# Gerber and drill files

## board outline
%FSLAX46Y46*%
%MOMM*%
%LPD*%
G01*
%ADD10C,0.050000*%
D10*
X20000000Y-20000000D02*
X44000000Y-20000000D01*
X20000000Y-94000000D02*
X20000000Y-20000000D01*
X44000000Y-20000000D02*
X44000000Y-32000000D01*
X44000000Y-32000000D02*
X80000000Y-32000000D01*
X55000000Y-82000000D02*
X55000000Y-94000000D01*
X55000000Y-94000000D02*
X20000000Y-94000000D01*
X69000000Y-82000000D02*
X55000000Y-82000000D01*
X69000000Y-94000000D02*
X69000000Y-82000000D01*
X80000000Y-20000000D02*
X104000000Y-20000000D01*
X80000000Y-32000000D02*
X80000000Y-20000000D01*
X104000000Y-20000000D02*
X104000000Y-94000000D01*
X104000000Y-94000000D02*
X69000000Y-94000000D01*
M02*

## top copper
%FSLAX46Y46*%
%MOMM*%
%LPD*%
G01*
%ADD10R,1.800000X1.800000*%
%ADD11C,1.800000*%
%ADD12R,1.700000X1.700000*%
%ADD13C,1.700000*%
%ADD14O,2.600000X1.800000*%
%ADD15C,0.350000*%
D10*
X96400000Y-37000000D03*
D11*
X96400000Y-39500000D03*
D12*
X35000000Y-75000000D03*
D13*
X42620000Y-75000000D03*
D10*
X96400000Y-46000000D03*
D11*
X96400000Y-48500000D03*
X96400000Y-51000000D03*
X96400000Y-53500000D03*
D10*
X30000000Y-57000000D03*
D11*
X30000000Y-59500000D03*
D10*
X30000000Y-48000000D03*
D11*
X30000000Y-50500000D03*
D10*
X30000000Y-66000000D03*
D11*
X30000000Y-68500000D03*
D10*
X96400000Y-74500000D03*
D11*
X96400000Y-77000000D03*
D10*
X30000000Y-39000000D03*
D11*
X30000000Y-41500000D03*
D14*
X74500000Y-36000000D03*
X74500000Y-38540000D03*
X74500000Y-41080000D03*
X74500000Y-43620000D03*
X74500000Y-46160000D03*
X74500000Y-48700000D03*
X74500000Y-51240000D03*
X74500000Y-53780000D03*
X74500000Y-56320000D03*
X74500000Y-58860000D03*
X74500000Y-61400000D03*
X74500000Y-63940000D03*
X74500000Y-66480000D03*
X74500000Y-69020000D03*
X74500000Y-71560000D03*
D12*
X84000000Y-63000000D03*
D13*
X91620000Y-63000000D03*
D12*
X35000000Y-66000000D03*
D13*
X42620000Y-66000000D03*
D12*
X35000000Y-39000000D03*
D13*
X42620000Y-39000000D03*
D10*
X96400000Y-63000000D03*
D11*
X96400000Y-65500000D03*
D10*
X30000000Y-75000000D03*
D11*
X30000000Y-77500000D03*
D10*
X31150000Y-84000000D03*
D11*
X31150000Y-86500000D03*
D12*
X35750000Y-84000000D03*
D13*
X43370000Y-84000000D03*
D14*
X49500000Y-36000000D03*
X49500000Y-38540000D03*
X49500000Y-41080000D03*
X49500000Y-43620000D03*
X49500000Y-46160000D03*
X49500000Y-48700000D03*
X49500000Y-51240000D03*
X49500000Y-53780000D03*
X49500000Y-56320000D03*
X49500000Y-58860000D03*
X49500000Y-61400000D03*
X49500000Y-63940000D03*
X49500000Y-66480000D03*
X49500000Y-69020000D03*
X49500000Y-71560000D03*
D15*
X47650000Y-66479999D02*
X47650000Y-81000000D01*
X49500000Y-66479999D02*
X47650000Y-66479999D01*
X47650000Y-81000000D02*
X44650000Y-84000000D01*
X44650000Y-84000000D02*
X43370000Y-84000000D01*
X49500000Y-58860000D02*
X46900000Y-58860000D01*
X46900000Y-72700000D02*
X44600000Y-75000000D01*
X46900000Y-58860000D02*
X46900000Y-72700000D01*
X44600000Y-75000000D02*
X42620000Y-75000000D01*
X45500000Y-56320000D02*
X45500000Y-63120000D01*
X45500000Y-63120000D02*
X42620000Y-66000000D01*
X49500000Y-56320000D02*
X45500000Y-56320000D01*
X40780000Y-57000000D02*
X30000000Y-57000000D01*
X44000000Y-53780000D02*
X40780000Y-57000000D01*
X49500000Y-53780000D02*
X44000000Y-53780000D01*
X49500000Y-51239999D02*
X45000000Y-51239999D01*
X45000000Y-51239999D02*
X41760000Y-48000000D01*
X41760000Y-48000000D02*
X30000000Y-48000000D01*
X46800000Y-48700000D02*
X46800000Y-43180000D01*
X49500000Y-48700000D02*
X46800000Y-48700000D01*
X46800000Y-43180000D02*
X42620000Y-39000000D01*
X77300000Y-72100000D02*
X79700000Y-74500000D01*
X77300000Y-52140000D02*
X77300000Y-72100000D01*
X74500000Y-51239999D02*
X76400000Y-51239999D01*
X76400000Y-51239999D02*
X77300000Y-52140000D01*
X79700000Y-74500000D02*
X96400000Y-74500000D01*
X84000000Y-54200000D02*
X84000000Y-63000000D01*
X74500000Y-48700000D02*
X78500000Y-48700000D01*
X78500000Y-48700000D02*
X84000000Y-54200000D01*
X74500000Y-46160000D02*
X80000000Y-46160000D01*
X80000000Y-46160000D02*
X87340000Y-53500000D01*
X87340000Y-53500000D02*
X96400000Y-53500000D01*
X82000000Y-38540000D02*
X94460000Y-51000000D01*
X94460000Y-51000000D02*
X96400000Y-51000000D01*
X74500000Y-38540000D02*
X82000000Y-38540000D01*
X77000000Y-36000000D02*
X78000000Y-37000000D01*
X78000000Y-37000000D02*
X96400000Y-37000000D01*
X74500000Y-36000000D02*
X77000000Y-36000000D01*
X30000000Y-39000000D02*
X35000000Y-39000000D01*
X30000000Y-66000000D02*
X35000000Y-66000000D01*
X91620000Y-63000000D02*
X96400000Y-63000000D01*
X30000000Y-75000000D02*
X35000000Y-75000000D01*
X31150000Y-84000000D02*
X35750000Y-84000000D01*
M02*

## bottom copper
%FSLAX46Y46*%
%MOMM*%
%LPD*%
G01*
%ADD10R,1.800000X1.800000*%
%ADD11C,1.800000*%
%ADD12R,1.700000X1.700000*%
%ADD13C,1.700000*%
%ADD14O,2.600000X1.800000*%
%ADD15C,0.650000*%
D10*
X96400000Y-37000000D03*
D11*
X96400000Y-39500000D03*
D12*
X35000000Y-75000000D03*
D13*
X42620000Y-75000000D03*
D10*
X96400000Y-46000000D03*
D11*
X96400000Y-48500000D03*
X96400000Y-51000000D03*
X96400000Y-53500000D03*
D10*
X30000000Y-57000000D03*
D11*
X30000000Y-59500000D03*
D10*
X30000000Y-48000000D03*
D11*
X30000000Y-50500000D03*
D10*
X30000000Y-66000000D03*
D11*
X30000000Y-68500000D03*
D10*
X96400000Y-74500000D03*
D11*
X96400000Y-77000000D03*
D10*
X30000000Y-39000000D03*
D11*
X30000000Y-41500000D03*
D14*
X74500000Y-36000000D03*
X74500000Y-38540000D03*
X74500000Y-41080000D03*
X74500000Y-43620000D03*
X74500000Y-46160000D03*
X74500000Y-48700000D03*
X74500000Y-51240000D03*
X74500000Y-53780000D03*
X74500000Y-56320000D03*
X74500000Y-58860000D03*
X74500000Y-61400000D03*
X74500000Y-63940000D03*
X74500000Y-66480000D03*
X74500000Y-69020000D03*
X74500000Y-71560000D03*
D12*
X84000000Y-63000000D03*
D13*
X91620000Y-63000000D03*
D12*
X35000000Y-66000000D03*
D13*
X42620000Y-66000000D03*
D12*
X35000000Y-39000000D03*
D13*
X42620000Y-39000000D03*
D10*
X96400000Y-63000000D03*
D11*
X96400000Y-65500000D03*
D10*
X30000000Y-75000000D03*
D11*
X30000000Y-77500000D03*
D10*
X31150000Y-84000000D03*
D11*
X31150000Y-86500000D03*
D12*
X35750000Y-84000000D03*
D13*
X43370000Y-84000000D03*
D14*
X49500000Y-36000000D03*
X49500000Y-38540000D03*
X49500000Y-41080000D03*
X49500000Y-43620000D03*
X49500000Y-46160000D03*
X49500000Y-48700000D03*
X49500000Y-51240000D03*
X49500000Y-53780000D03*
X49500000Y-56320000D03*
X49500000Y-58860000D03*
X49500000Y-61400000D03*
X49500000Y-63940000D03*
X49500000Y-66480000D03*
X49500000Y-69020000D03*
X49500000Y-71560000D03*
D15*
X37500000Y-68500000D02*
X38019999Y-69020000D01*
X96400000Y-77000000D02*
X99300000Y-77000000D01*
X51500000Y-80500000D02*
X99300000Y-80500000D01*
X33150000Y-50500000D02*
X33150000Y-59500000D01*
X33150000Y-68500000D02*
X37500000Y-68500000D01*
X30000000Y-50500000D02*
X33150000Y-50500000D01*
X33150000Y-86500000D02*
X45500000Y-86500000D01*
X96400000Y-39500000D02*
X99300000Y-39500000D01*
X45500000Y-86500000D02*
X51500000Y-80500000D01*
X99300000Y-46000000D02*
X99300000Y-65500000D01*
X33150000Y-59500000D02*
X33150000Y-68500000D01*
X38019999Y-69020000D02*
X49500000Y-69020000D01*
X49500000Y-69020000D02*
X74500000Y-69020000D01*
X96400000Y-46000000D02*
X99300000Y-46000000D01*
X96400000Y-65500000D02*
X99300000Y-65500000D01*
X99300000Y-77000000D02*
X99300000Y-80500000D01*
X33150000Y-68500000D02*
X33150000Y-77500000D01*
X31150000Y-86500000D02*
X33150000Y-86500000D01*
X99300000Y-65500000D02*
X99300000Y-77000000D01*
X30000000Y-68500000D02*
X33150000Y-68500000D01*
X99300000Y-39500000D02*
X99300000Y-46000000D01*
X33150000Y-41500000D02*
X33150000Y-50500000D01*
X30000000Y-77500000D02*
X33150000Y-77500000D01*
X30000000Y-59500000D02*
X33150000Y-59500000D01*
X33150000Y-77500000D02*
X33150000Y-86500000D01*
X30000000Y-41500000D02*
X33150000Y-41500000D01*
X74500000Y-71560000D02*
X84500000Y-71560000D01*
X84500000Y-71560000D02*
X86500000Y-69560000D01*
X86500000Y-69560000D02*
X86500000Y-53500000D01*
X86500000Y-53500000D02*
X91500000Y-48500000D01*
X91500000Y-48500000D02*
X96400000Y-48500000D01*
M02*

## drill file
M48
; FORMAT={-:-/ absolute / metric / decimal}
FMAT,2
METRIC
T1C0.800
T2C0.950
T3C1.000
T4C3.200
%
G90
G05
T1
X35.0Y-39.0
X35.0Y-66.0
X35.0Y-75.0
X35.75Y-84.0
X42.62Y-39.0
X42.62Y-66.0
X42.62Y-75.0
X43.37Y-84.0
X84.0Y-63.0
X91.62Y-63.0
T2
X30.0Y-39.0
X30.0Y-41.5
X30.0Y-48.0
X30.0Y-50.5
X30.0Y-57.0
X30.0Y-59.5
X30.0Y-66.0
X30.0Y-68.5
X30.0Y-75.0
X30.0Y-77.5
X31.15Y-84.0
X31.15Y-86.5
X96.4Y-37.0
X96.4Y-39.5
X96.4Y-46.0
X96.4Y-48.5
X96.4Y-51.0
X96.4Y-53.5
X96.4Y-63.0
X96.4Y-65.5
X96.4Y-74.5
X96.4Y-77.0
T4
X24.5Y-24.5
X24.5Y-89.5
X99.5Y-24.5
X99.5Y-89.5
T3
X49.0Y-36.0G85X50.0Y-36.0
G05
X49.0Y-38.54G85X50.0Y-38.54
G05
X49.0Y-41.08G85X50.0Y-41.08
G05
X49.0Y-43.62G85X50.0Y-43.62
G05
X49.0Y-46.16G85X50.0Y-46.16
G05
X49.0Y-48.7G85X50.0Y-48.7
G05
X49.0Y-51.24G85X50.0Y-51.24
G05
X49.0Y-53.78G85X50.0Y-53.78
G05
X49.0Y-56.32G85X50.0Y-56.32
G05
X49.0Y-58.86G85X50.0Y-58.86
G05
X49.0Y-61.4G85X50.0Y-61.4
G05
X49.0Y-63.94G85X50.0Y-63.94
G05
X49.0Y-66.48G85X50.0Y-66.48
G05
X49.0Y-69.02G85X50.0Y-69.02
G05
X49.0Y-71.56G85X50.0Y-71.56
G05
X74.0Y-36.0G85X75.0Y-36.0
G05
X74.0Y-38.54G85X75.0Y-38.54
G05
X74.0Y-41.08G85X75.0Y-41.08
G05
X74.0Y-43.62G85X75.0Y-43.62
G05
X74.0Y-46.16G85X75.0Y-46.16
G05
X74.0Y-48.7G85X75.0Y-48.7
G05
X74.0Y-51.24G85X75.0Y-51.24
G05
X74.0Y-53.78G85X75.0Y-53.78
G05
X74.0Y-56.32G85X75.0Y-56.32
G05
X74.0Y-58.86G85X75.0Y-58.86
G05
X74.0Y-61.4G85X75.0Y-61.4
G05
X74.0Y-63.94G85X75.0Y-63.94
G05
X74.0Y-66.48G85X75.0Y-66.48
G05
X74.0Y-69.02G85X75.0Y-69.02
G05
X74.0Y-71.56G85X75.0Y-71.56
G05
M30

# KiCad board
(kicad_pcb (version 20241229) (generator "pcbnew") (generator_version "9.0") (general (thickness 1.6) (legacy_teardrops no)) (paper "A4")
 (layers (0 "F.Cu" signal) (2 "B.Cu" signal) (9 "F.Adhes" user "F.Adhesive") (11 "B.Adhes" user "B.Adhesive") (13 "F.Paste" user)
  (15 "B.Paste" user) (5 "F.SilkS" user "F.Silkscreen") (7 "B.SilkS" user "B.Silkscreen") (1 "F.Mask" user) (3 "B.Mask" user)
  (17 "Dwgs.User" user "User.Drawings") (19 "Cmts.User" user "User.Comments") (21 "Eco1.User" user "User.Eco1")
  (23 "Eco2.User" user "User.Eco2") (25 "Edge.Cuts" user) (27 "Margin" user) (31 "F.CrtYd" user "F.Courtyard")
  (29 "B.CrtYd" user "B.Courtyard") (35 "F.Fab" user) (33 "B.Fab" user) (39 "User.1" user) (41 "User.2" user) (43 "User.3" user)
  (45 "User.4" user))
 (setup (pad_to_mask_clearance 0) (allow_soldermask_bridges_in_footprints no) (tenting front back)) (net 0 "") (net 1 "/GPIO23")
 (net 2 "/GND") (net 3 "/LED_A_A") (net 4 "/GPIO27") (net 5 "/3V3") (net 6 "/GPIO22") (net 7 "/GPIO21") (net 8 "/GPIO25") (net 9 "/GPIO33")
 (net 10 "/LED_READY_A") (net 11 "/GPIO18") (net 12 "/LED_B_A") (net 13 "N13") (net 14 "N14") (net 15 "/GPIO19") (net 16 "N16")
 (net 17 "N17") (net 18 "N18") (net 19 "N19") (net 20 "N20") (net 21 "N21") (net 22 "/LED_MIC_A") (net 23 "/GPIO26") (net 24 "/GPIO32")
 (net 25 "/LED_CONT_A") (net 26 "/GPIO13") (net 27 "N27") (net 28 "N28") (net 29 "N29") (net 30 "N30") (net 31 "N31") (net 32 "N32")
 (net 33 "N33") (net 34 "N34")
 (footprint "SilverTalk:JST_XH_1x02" (layer "F.Cu") (at 96.4 37)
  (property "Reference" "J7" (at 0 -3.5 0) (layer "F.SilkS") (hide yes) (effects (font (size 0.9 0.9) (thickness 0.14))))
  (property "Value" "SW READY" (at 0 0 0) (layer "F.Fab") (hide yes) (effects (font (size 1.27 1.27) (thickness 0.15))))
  (pad "1" thru_hole rect (at 0 0) (size 1.8 1.8) (drill 0.95) (layers "*.Cu" "*.Mask") (remove_unused_layers no) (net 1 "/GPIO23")
   (thermal_bridge_angle 45))
  (pad "2" thru_hole circle (at 0 2.5) (size 1.8 1.8) (drill 0.95) (layers "*.Cu" "*.Mask") (remove_unused_layers no) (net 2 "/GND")))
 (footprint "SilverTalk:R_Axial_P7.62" (layer "F.Cu") (at 35 75)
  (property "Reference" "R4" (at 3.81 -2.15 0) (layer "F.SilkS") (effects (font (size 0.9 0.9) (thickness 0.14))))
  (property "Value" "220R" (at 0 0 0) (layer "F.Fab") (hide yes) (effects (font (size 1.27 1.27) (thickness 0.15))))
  (pad "1" thru_hole rect (at 0 0) (size 1.7 1.7) (drill 0.8) (layers "*.Cu" "*.Mask") (remove_unused_layers no) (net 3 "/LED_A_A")
   (thermal_bridge_angle 45))
  (pad "2" thru_hole circle (at 7.62 0) (size 1.7 1.7) (drill 0.8) (layers "*.Cu" "*.Mask") (remove_unused_layers no) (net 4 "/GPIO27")))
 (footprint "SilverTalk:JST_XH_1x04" (layer "F.Cu") (at 96.4 46)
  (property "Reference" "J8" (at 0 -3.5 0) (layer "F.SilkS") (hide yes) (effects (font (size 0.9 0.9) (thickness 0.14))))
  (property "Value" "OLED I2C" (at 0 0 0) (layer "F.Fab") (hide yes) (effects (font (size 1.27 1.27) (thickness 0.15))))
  (pad "1" thru_hole rect (at 0 0) (size 1.8 1.8) (drill 0.95) (layers "*.Cu" "*.Mask") (remove_unused_layers no) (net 2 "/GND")
   (thermal_bridge_angle 45))
  (pad "2" thru_hole circle (at 0 2.5) (size 1.8 1.8) (drill 0.95) (layers "*.Cu" "*.Mask") (remove_unused_layers no) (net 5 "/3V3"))
  (pad "3" thru_hole circle (at 0 5) (size 1.8 1.8) (drill 0.95) (layers "*.Cu" "*.Mask") (remove_unused_layers no) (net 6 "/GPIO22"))
  (pad "4" thru_hole circle (at 0 7.5) (size 1.8 1.8) (drill 0.95) (layers "*.Cu" "*.Mask") (remove_unused_layers no) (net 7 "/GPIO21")))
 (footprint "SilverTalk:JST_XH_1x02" (layer "F.Cu") (at 30 57)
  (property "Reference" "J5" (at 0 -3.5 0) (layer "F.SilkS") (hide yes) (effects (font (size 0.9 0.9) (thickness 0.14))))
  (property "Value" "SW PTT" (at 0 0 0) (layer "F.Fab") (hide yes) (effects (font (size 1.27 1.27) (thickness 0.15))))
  (pad "1" thru_hole rect (at 0 0) (size 1.8 1.8) (drill 0.95) (layers "*.Cu" "*.Mask") (remove_unused_layers no) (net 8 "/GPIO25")
   (thermal_bridge_angle 45))
  (pad "2" thru_hole circle (at 0 2.5) (size 1.8 1.8) (drill 0.95) (layers "*.Cu" "*.Mask") (remove_unused_layers no) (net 2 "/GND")))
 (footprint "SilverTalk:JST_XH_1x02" (layer "F.Cu") (at 30 48)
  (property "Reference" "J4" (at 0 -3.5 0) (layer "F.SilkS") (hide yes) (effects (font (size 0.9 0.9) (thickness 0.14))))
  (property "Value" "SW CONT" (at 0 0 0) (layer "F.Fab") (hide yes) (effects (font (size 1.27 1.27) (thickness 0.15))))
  (pad "1" thru_hole rect (at 0 0) (size 1.8 1.8) (drill 0.95) (layers "*.Cu" "*.Mask") (remove_unused_layers no) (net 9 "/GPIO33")
   (thermal_bridge_angle 45))
  (pad "2" thru_hole circle (at 0 2.5) (size 1.8 1.8) (drill 0.95) (layers "*.Cu" "*.Mask") (remove_unused_layers no) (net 2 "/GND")))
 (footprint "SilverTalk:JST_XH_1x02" (layer "F.Cu") (at 30 66)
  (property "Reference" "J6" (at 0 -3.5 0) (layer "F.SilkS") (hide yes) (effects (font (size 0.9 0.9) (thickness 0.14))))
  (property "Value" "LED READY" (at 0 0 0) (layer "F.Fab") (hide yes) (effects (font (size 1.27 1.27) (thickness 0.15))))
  (pad "1" thru_hole rect (at 0 0) (size 1.8 1.8) (drill 0.95) (layers "*.Cu" "*.Mask") (remove_unused_layers no) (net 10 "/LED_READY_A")
   (thermal_bridge_angle 45))
  (pad "2" thru_hole circle (at 0 2.5) (size 1.8 1.8) (drill 0.95) (layers "*.Cu" "*.Mask") (remove_unused_layers no) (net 2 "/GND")))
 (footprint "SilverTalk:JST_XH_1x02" (layer "F.Cu") (at 96.4 74.5)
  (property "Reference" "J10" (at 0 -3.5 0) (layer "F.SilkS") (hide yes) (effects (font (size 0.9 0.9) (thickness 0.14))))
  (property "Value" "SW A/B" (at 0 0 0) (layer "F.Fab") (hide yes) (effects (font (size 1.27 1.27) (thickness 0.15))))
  (pad "1" thru_hole rect (at 0 0) (size 1.8 1.8) (drill 0.95) (layers "*.Cu" "*.Mask") (remove_unused_layers no) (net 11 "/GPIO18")
   (thermal_bridge_angle 45))
  (pad "2" thru_hole circle (at 0 2.5) (size 1.8 1.8) (drill 0.95) (layers "*.Cu" "*.Mask") (remove_unused_layers no) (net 2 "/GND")))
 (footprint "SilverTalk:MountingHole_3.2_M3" (layer "F.Cu") (at 99.5 24.5)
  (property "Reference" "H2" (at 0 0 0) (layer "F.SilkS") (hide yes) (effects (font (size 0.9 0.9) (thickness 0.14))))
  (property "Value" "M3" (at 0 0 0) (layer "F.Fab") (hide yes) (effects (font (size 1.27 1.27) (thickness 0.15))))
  (pad "" np_thru_hole circle (at 0 0) (size 3.2 3.2) (drill 3.2) (layers "*.Cu" "*.Mask")))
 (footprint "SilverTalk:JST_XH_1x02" (layer "F.Cu") (at 30 39)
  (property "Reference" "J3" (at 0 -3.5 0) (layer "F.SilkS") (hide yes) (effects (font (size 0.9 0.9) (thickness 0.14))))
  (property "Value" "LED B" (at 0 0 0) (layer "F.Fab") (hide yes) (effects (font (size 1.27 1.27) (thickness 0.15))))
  (pad "1" thru_hole rect (at 0 0) (size 1.8 1.8) (drill 0.95) (layers "*.Cu" "*.Mask") (remove_unused_layers no) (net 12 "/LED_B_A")
   (thermal_bridge_angle 45))
  (pad "2" thru_hole circle (at 0 2.5) (size 1.8 1.8) (drill 0.95) (layers "*.Cu" "*.Mask") (remove_unused_layers no) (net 2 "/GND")))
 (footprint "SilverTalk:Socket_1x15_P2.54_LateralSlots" (layer "F.Cu") (at 74.5 36)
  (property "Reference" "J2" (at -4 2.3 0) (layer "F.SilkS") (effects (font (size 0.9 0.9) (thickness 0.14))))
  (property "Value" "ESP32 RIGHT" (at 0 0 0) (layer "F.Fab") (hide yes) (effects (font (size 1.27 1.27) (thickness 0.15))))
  (pad "1" thru_hole oval (at 0 0) (size 2.6 1.8) (drill oval 2 1) (layers "*.Cu" "*.Mask") (remove_unused_layers no) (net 1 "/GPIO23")
   (thermal_bridge_angle 45))
  (pad "2" thru_hole oval (at 0 2.54) (size 2.6 1.8) (drill oval 2 1) (layers "*.Cu" "*.Mask") (remove_unused_layers no) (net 6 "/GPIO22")
   (thermal_bridge_angle 45))
  (pad "3" thru_hole oval (at 0 5.08) (size 2.6 1.8) (drill oval 2 1) (layers "*.Cu" "*.Mask") (remove_unused_layers no) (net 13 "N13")
   (thermal_bridge_angle 45))
  (pad "4" thru_hole oval (at 0 7.62) (size 2.6 1.8) (drill oval 2 1) (layers "*.Cu" "*.Mask") (remove_unused_layers no) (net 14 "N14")
   (thermal_bridge_angle 45))
  (pad "5" thru_hole oval (at 0 10.16) (size 2.6 1.8) (drill oval 2 1) (layers "*.Cu" "*.Mask") (remove_unused_layers no) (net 7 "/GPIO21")
   (thermal_bridge_angle 45))
  (pad "6" thru_hole oval (at 0 12.7) (size 2.6 1.8) (drill oval 2 1) (layers "*.Cu" "*.Mask") (remove_unused_layers no) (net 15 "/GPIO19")
   (thermal_bridge_angle 45))
  (pad "7" thru_hole oval (at 0 15.24) (size 2.6 1.8) (drill oval 2 1) (layers "*.Cu" "*.Mask") (remove_unused_layers no) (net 11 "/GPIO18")
   (thermal_bridge_angle 45))
  (pad "8" thru_hole oval (at 0 17.78) (size 2.6 1.8) (drill oval 2 1) (layers "*.Cu" "*.Mask") (remove_unused_layers no) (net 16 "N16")
   (thermal_bridge_angle 45))
  (pad "9" thru_hole oval (at 0 20.32) (size 2.6 1.8) (drill oval 2 1) (layers "*.Cu" "*.Mask") (remove_unused_layers no) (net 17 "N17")
   (thermal_bridge_angle 45))
  (pad "10" thru_hole oval (at 0 22.86) (size 2.6 1.8) (drill oval 2 1) (layers "*.Cu" "*.Mask") (remove_unused_layers no) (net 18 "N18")
   (thermal_bridge_angle 45))
  (pad "11" thru_hole oval (at 0 25.4) (size 2.6 1.8) (drill oval 2 1) (layers "*.Cu" "*.Mask") (remove_unused_layers no) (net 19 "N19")
   (thermal_bridge_angle 45))
  (pad "12" thru_hole oval (at 0 27.94) (size 2.6 1.8) (drill oval 2 1) (layers "*.Cu" "*.Mask") (remove_unused_layers no) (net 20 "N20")
   (thermal_bridge_angle 45))
  (pad "13" thru_hole oval (at 0 30.48) (size 2.6 1.8) (drill oval 2 1) (layers "*.Cu" "*.Mask") (remove_unused_layers no) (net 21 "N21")
   (thermal_bridge_angle 45))
  (pad "14" thru_hole oval (at 0 33.02) (size 2.6 1.8) (drill oval 2 1) (layers "*.Cu" "*.Mask") (remove_unused_layers no) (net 2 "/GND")
   (thermal_bridge_angle 45))
  (pad "15" thru_hole oval (at 0 35.56) (size 2.6 1.8) (drill oval 2 1) (layers "*.Cu" "*.Mask") (remove_unused_layers no) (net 5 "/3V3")
   (thermal_bridge_angle 45)))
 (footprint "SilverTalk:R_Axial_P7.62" (layer "F.Cu") (at 84 63)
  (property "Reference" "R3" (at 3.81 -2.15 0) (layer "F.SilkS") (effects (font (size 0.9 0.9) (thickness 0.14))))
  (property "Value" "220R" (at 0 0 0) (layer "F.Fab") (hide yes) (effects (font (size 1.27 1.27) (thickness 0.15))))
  (pad "1" thru_hole rect (at 0 0) (size 1.7 1.7) (drill 0.8) (layers "*.Cu" "*.Mask") (remove_unused_layers no) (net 15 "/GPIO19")
   (thermal_bridge_angle 45))
  (pad "2" thru_hole circle (at 7.62 0) (size 1.7 1.7) (drill 0.8) (layers "*.Cu" "*.Mask") (remove_unused_layers no) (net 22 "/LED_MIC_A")))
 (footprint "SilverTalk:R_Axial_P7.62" (layer "F.Cu") (at 35 66)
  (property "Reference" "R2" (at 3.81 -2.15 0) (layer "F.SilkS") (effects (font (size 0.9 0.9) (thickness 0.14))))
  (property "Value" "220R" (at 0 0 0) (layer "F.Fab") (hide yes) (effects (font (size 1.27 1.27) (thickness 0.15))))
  (pad "1" thru_hole rect (at 0 0) (size 1.7 1.7) (drill 0.8) (layers "*.Cu" "*.Mask") (remove_unused_layers no) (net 10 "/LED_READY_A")
   (thermal_bridge_angle 45))
  (pad "2" thru_hole circle (at 7.62 0) (size 1.7 1.7) (drill 0.8) (layers "*.Cu" "*.Mask") (remove_unused_layers no) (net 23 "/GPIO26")))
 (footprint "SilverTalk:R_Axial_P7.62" (layer "F.Cu") (at 35 39)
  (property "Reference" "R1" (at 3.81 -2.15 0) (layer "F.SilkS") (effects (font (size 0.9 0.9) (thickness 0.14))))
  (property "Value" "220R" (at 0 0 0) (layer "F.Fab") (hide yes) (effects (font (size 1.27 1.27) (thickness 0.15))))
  (pad "1" thru_hole rect (at 0 0) (size 1.7 1.7) (drill 0.8) (layers "*.Cu" "*.Mask") (remove_unused_layers no) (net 12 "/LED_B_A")
   (thermal_bridge_angle 45))
  (pad "2" thru_hole circle (at 7.62 0) (size 1.7 1.7) (drill 0.8) (layers "*.Cu" "*.Mask") (remove_unused_layers no) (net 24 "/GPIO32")))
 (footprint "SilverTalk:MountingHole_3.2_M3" (layer "F.Cu") (at 99.5 89.5)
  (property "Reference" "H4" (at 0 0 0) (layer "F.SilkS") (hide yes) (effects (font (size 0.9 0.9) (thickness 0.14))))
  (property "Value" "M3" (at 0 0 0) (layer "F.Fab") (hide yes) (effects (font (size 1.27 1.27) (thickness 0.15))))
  (pad "" np_thru_hole circle (at 0 0) (size 3.2 3.2) (drill 3.2) (layers "*.Cu" "*.Mask")))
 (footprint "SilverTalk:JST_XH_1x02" (layer "F.Cu") (at 96.4 63)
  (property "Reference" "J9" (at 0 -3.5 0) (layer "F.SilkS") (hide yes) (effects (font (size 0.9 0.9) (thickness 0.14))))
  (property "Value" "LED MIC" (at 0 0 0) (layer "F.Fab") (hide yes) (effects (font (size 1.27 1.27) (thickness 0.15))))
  (pad "1" thru_hole rect (at 0 0) (size 1.8 1.8) (drill 0.95) (layers "*.Cu" "*.Mask") (remove_unused_layers no) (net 22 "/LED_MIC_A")
   (thermal_bridge_angle 45))
  (pad "2" thru_hole circle (at 0 2.5) (size 1.8 1.8) (drill 0.95) (layers "*.Cu" "*.Mask") (remove_unused_layers no) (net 2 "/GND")))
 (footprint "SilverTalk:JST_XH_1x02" (layer "F.Cu") (at 30 75)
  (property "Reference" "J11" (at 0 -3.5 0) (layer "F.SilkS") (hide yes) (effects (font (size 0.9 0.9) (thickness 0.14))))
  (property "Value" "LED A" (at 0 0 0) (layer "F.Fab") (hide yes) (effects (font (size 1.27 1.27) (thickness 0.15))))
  (pad "1" thru_hole rect (at 0 0) (size 1.8 1.8) (drill 0.95) (layers "*.Cu" "*.Mask") (remove_unused_layers no) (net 3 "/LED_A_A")
   (thermal_bridge_angle 45))
  (pad "2" thru_hole circle (at 0 2.5) (size 1.8 1.8) (drill 0.95) (layers "*.Cu" "*.Mask") (remove_unused_layers no) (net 2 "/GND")))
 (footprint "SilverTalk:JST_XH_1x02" (layer "F.Cu") (at 31.15 84)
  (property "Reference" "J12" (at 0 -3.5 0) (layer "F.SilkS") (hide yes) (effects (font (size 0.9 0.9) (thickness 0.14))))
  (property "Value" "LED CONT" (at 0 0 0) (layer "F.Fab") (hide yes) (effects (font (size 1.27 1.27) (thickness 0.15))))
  (pad "1" thru_hole rect (at 0 0) (size 1.8 1.8) (drill 0.95) (layers "*.Cu" "*.Mask") (remove_unused_layers no) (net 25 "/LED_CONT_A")
   (thermal_bridge_angle 45))
  (pad "2" thru_hole circle (at 0 2.5) (size 1.8 1.8) (drill 0.95) (layers "*.Cu" "*.Mask") (remove_unused_layers no) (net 2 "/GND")))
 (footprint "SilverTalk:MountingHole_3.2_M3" (layer "F.Cu") (at 24.5 24.5)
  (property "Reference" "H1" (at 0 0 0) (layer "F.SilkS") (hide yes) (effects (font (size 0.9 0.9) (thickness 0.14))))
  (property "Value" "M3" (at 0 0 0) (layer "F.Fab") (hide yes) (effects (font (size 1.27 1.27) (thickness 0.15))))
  (pad "" np_thru_hole circle (at 0 0) (size 3.2 3.2) (drill 3.2) (layers "*.Cu" "*.Mask")))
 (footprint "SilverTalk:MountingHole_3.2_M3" (layer "F.Cu") (at 24.5 89.5)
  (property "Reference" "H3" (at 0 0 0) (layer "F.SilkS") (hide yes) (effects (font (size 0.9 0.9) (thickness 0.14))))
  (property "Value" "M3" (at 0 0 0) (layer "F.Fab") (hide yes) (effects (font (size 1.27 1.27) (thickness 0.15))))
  (pad "" np_thru_hole circle (at 0 0) (size 3.2 3.2) (drill 3.2) (layers "*.Cu" "*.Mask")))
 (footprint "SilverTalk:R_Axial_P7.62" (layer "F.Cu") (at 35.75 84)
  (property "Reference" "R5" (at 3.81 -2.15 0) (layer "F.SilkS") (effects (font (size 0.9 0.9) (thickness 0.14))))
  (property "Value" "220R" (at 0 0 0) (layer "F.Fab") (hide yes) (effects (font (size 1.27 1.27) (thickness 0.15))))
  (pad "1" thru_hole rect (at 0 0) (size 1.7 1.7) (drill 0.8) (layers "*.Cu" "*.Mask") (remove_unused_layers no) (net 25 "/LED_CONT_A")
   (thermal_bridge_angle 45))
  (pad "2" thru_hole circle (at 7.62 0) (size 1.7 1.7) (drill 0.8) (layers "*.Cu" "*.Mask") (remove_unused_layers no) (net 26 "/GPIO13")))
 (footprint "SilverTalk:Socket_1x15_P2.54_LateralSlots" (layer "F.Cu") (at 49.5 36)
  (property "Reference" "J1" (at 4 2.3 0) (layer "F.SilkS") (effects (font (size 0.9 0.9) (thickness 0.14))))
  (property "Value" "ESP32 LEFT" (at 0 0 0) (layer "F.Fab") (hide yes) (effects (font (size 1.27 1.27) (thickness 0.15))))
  (pad "1" thru_hole oval (at 0 0) (size 2.6 1.8) (drill oval 2 1) (layers "*.Cu" "*.Mask") (remove_unused_layers no) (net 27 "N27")
   (thermal_bridge_angle 45))
  (pad "2" thru_hole oval (at 0 2.54) (size 2.6 1.8) (drill oval 2 1) (layers "*.Cu" "*.Mask") (remove_unused_layers no) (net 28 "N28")
   (thermal_bridge_angle 45))
  (pad "3" thru_hole oval (at 0 5.08) (size 2.6 1.8) (drill oval 2 1) (layers "*.Cu" "*.Mask") (remove_unused_layers no) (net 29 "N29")
   (thermal_bridge_angle 45))
  (pad "4" thru_hole oval (at 0 7.62) (size 2.6 1.8) (drill oval 2 1) (layers "*.Cu" "*.Mask") (remove_unused_layers no) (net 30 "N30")
   (thermal_bridge_angle 45))
  (pad "5" thru_hole oval (at 0 10.16) (size 2.6 1.8) (drill oval 2 1) (layers "*.Cu" "*.Mask") (remove_unused_layers no) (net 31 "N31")
   (thermal_bridge_angle 45))
  (pad "6" thru_hole oval (at 0 12.7) (size 2.6 1.8) (drill oval 2 1) (layers "*.Cu" "*.Mask") (remove_unused_layers no) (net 24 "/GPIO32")
   (thermal_bridge_angle 45))
  (pad "7" thru_hole oval (at 0 15.24) (size 2.6 1.8) (drill oval 2 1) (layers "*.Cu" "*.Mask") (remove_unused_layers no) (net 9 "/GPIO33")
   (thermal_bridge_angle 45))
  (pad "8" thru_hole oval (at 0 17.78) (size 2.6 1.8) (drill oval 2 1) (layers "*.Cu" "*.Mask") (remove_unused_layers no) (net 8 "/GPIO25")
   (thermal_bridge_angle 45))
  (pad "9" thru_hole oval (at 0 20.32) (size 2.6 1.8) (drill oval 2 1) (layers "*.Cu" "*.Mask") (remove_unused_layers no) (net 23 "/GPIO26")
   (thermal_bridge_angle 45))
  (pad "10" thru_hole oval (at 0 22.86) (size 2.6 1.8) (drill oval 2 1) (layers "*.Cu" "*.Mask") (remove_unused_layers no) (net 4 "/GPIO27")
   (thermal_bridge_angle 45))
  (pad "11" thru_hole oval (at 0 25.4) (size 2.6 1.8) (drill oval 2 1) (layers "*.Cu" "*.Mask") (remove_unused_layers no) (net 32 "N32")
   (thermal_bridge_angle 45))
  (pad "12" thru_hole oval (at 0 27.94) (size 2.6 1.8) (drill oval 2 1) (layers "*.Cu" "*.Mask") (remove_unused_layers no) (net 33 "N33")
   (thermal_bridge_angle 45))
  (pad "13" thru_hole oval (at 0 30.48) (size 2.6 1.8) (drill oval 2 1) (layers "*.Cu" "*.Mask") (remove_unused_layers no)
   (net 26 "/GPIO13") (thermal_bridge_angle 45))
  (pad "14" thru_hole oval (at 0 33.02) (size 2.6 1.8) (drill oval 2 1) (layers "*.Cu" "*.Mask") (remove_unused_layers no) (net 2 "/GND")
   (thermal_bridge_angle 45))
  (pad "15" thru_hole oval (at 0 35.56) (size 2.6 1.8) (drill oval 2 1) (layers "*.Cu" "*.Mask") (remove_unused_layers no) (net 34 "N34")
   (thermal_bridge_angle 45)))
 (gr_line (start 20 20) (end 44 20) (stroke (width 0.05) (type default)) (layer "Edge.Cuts"))
 (gr_line (start 20 94) (end 20 20) (stroke (width 0.05) (type default)) (layer "Edge.Cuts"))
 (gr_line (start 44 20) (end 44 32) (stroke (width 0.05) (type default)) (layer "Edge.Cuts"))
 (gr_line (start 44 32) (end 80 32) (stroke (width 0.05) (type default)) (layer "Edge.Cuts"))
 (gr_line (start 55 82) (end 55 94) (stroke (width 0.05) (type default)) (layer "Edge.Cuts"))
 (gr_line (start 55 94) (end 20 94) (stroke (width 0.05) (type default)) (layer "Edge.Cuts"))
 (gr_line (start 69 82) (end 55 82) (stroke (width 0.05) (type default)) (layer "Edge.Cuts"))
 (gr_line (start 69 94) (end 69 82) (stroke (width 0.05) (type default)) (layer "Edge.Cuts"))
 (gr_line (start 80 20) (end 104 20) (stroke (width 0.05) (type default)) (layer "Edge.Cuts"))
 (gr_line (start 80 32) (end 80 20) (stroke (width 0.05) (type default)) (layer "Edge.Cuts"))
 (gr_line (start 104 20) (end 104 94) (stroke (width 0.05) (type default)) (layer "Edge.Cuts"))
 (gr_line (start 104 94) (end 69 94) (stroke (width 0.05) (type default)) (layer "Edge.Cuts"))
 (segment (start 37.5 68.5) (end 38.019999 69.02) (width 0.65) (layer "B.Cu") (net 2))
 (segment (start 96.4 77) (end 99.3 77) (width 0.65) (layer "B.Cu") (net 2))
 (segment (start 51.5 80.5) (end 99.3 80.5) (width 0.65) (layer "B.Cu") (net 2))
 (segment (start 33.15 50.5) (end 33.15 59.5) (width 0.65) (layer "B.Cu") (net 2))
 (segment (start 33.15 68.5) (end 37.5 68.5) (width 0.65) (layer "B.Cu") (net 2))
 (segment (start 30 50.5) (end 33.15 50.5) (width 0.65) (layer "B.Cu") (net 2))
 (segment (start 33.15 86.5) (end 45.5 86.5) (width 0.65) (layer "B.Cu") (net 2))
 (segment (start 96.4 39.5) (end 99.3 39.5) (width 0.65) (layer "B.Cu") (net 2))
 (segment (start 45.5 86.5) (end 51.5 80.5) (width 0.65) (layer "B.Cu") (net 2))
 (segment (start 99.3 46) (end 99.3 65.5) (width 0.65) (layer "B.Cu") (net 2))
 (segment (start 33.15 59.5) (end 33.15 68.5) (width 0.65) (layer "B.Cu") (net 2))
 (segment (start 38.019999 69.02) (end 49.5 69.02) (width 0.65) (layer "B.Cu") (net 2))
 (segment (start 49.5 69.02) (end 74.5 69.02) (width 0.65) (layer "B.Cu") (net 2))
 (segment (start 96.4 46) (end 99.3 46) (width 0.65) (layer "B.Cu") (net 2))
 (segment (start 96.4 65.5) (end 99.3 65.5) (width 0.65) (layer "B.Cu") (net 2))
 (segment (start 99.3 77) (end 99.3 80.5) (width 0.65) (layer "B.Cu") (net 2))
 (segment (start 33.15 68.5) (end 33.15 77.5) (width 0.65) (layer "B.Cu") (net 2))
 (segment (start 31.15 86.5) (end 33.15 86.5) (width 0.65) (layer "B.Cu") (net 2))
 (segment (start 99.3 65.5) (end 99.3 77) (width 0.65) (layer "B.Cu") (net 2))
 (segment (start 30 68.5) (end 33.15 68.5) (width 0.65) (layer "B.Cu") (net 2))
 (segment (start 99.3 39.5) (end 99.3 46) (width 0.65) (layer "B.Cu") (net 2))
 (segment (start 33.15 41.5) (end 33.15 50.5) (width 0.65) (layer "B.Cu") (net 2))
 (segment (start 30 77.5) (end 33.15 77.5) (width 0.65) (layer "B.Cu") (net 2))
 (segment (start 30 59.5) (end 33.15 59.5) (width 0.65) (layer "B.Cu") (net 2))
 (segment (start 33.15 77.5) (end 33.15 86.5) (width 0.65) (layer "B.Cu") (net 2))
 (segment (start 30 41.5) (end 33.15 41.5) (width 0.65) (layer "B.Cu") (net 2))
 (segment (start 47.65 66.479999) (end 47.65 81) (width 0.35) (layer "F.Cu") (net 26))
 (segment (start 49.5 66.479999) (end 47.65 66.479999) (width 0.35) (layer "F.Cu") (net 26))
 (segment (start 47.65 81) (end 44.65 84) (width 0.35) (layer "F.Cu") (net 26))
 (segment (start 44.65 84) (end 43.37 84) (width 0.35) (layer "F.Cu") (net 26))
 (segment (start 49.5 58.86) (end 46.9 58.86) (width 0.35) (layer "F.Cu") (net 4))
 (segment (start 46.9 72.7) (end 44.6 75) (width 0.35) (layer "F.Cu") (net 4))
 (segment (start 46.9 58.86) (end 46.9 72.7) (width 0.35) (layer "F.Cu") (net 4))
 (segment (start 44.6 75) (end 42.62 75) (width 0.35) (layer "F.Cu") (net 4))
 (segment (start 45.5 56.32) (end 45.5 63.12) (width 0.35) (layer "F.Cu") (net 23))
 (segment (start 45.5 63.12) (end 42.62 66) (width 0.35) (layer "F.Cu") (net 23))
 (segment (start 49.5 56.32) (end 45.5 56.32) (width 0.35) (layer "F.Cu") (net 23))
 (segment (start 40.78 57) (end 30 57) (width 0.35) (layer "F.Cu") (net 8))
 (segment (start 44 53.78) (end 40.78 57) (width 0.35) (layer "F.Cu") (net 8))
 (segment (start 49.5 53.78) (end 44 53.78) (width 0.35) (layer "F.Cu") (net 8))
 (segment (start 49.5 51.239999) (end 45 51.239999) (width 0.35) (layer "F.Cu") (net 9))
 (segment (start 45 51.239999) (end 41.76 48) (width 0.35) (layer "F.Cu") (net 9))
 (segment (start 41.76 48) (end 30 48) (width 0.35) (layer "F.Cu") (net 9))
 (segment (start 46.8 48.7) (end 46.8 43.18) (width 0.35) (layer "F.Cu") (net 24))
 (segment (start 49.5 48.7) (end 46.8 48.7) (width 0.35) (layer "F.Cu") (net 24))
 (segment (start 46.8 43.18) (end 42.62 39) (width 0.35) (layer "F.Cu") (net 24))
 (segment (start 74.5 71.56) (end 84.5 71.56) (width 0.65) (layer "B.Cu") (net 5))
 (segment (start 84.5 71.56) (end 86.5 69.56) (width 0.65) (layer "B.Cu") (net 5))
 (segment (start 86.5 69.56) (end 86.5 53.5) (width 0.65) (layer "B.Cu") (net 5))
 (segment (start 86.5 53.5) (end 91.5 48.5) (width 0.65) (layer "B.Cu") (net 5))
 (segment (start 91.5 48.5) (end 96.4 48.5) (width 0.65) (layer "B.Cu") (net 5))
 (segment (start 77.3 72.1) (end 79.7 74.5) (width 0.35) (layer "F.Cu") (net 11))
 (segment (start 77.3 52.14) (end 77.3 72.1) (width 0.35) (layer "F.Cu") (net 11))
 (segment (start 74.5 51.239999) (end 76.4 51.239999) (width 0.35) (layer "F.Cu") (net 11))
 (segment (start 76.4 51.239999) (end 77.3 52.14) (width 0.35) (layer "F.Cu") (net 11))
 (segment (start 79.7 74.5) (end 96.4 74.5) (width 0.35) (layer "F.Cu") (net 11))
 (segment (start 84 54.2) (end 84 63) (width 0.35) (layer "F.Cu") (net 15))
 (segment (start 74.5 48.7) (end 78.5 48.7) (width 0.35) (layer "F.Cu") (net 15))
 (segment (start 78.5 48.7) (end 84 54.2) (width 0.35) (layer "F.Cu") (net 15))
 (segment (start 74.5 46.16) (end 80 46.16) (width 0.35) (layer "F.Cu") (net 7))
 (segment (start 80 46.16) (end 87.34 53.5) (width 0.35) (layer "F.Cu") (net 7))
 (segment (start 87.34 53.5) (end 96.4 53.5) (width 0.35) (layer "F.Cu") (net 7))
 (segment (start 82 38.54) (end 94.46 51) (width 0.35) (layer "F.Cu") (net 6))
 (segment (start 94.46 51) (end 96.4 51) (width 0.35) (layer "F.Cu") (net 6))
 (segment (start 74.5 38.54) (end 82 38.54) (width 0.35) (layer "F.Cu") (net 6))
 (segment (start 77 36) (end 78 37) (width 0.35) (layer "F.Cu") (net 1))
 (segment (start 78 37) (end 96.4 37) (width 0.35) (layer "F.Cu") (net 1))
 (segment (start 74.5 36) (end 77 36) (width 0.35) (layer "F.Cu") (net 1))
 (segment (start 30 39) (end 35 39) (width 0.35) (layer "F.Cu") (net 12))
 (segment (start 30 66) (end 35 66) (width 0.35) (layer "F.Cu") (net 10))
 (segment (start 91.62 63) (end 96.4 63) (width 0.35) (layer "F.Cu") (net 22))
 (segment (start 30 75) (end 35 75) (width 0.35) (layer "F.Cu") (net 3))
 (segment (start 31.15 84) (end 35.75 84) (width 0.35) (layer "F.Cu") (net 25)))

